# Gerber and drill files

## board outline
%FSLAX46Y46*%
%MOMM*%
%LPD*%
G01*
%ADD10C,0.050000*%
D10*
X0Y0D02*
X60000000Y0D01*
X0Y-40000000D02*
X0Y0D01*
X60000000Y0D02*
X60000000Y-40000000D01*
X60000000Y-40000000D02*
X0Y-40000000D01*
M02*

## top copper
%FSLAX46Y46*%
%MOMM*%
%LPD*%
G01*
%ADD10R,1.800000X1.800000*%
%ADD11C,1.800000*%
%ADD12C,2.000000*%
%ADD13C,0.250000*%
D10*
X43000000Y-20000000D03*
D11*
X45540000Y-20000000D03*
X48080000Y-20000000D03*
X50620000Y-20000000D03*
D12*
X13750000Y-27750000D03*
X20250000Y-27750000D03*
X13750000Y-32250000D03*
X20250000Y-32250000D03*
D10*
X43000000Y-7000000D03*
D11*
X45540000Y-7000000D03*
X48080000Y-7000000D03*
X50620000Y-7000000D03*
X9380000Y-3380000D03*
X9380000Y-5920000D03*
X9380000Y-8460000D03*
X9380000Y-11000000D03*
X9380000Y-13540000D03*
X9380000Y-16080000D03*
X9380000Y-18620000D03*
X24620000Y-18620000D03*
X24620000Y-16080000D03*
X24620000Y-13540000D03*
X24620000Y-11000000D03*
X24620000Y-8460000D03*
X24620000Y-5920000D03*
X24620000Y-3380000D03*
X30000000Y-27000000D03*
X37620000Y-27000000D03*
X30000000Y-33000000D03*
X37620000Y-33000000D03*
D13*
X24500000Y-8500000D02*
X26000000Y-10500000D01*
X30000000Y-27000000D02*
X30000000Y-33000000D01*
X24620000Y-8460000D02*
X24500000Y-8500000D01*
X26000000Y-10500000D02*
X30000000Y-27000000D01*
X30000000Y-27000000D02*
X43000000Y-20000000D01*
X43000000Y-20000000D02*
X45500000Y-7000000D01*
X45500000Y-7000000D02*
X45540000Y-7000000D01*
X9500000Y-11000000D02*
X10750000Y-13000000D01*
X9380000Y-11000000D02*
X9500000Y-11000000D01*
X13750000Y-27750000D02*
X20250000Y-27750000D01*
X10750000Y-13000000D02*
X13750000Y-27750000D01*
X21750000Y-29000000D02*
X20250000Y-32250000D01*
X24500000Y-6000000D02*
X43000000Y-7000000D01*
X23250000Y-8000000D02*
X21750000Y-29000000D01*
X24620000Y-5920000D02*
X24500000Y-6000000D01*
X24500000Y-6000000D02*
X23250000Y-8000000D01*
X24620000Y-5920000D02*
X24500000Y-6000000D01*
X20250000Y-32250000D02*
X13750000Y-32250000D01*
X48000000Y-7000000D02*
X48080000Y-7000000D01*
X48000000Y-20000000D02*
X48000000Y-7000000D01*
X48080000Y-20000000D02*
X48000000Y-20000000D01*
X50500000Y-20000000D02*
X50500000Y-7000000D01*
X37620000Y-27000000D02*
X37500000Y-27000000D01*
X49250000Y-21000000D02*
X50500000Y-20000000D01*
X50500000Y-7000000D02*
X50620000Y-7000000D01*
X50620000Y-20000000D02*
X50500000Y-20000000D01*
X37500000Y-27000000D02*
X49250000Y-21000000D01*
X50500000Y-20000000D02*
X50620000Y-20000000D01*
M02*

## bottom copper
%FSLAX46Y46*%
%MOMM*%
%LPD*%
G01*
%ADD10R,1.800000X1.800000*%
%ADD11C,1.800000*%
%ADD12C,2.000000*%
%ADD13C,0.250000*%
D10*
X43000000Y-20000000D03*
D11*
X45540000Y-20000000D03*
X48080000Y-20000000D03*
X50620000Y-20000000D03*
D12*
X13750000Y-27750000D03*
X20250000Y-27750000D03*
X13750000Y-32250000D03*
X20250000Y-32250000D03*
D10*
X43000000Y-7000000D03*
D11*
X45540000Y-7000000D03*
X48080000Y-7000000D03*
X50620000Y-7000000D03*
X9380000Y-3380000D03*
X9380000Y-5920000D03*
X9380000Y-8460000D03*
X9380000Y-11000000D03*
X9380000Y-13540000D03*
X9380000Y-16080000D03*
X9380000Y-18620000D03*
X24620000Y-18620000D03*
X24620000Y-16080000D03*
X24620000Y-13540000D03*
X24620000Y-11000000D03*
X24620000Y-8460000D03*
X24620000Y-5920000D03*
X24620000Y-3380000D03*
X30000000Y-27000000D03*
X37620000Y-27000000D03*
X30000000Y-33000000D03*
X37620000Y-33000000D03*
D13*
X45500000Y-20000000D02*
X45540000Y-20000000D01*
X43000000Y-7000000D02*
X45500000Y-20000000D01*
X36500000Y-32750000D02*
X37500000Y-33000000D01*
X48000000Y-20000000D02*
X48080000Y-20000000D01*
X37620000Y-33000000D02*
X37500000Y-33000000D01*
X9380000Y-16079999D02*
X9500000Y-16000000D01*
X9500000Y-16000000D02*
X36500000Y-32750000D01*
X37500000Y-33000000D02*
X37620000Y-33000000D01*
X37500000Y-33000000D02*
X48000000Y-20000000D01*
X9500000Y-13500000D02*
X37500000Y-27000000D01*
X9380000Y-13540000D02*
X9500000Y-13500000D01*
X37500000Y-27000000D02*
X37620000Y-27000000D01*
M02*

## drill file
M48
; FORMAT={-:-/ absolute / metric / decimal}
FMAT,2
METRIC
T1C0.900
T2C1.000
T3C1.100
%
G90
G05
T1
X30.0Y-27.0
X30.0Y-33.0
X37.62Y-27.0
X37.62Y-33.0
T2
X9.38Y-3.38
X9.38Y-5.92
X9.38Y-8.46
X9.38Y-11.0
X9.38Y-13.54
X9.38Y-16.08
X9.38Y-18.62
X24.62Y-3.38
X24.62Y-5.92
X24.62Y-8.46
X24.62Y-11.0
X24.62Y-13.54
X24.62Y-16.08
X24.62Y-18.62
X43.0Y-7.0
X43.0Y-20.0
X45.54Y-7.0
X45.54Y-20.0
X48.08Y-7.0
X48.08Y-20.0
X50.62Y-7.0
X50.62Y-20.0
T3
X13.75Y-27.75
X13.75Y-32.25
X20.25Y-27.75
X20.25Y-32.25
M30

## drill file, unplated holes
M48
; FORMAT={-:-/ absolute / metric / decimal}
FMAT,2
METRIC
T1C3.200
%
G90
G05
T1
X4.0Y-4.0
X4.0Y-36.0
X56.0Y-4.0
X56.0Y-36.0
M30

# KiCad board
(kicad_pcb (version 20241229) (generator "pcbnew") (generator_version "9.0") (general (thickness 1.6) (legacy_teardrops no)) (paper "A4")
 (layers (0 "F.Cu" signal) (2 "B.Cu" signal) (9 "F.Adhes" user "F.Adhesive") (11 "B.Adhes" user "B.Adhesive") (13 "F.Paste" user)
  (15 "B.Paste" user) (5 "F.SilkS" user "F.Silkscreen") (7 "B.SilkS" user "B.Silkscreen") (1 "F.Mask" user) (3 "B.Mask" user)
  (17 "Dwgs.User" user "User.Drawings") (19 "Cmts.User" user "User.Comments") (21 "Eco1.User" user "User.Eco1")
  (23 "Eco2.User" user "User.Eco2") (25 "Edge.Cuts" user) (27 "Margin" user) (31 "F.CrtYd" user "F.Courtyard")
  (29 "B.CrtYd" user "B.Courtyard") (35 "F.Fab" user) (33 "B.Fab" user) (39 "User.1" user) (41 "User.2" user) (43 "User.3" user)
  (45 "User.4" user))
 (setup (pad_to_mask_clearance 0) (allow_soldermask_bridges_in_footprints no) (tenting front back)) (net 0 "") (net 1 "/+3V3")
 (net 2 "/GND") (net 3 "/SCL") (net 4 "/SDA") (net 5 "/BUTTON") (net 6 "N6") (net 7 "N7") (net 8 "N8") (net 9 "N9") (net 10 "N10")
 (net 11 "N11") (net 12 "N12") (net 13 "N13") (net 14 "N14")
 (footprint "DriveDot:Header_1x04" (layer "F.Cu") (at 43 20)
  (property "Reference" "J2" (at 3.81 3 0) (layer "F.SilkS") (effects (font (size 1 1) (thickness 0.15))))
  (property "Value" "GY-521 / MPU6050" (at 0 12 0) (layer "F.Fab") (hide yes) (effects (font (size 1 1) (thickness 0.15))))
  (pad "1" thru_hole rect (at 0 0) (size 1.8 1.8) (drill 1) (layers "*.Cu" "*.Mask") (remove_unused_layers no) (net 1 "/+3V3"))
  (pad "2" thru_hole circle (at 2.54 0) (size 1.8 1.8) (drill 1) (layers "*.Cu" "*.Mask") (remove_unused_layers no) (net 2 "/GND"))
  (pad "3" thru_hole circle (at 5.08 0) (size 1.8 1.8) (drill 1) (layers "*.Cu" "*.Mask") (remove_unused_layers no) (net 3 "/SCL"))
  (pad "4" thru_hole circle (at 7.62 0) (size 1.8 1.8) (drill 1) (layers "*.Cu" "*.Mask") (remove_unused_layers no) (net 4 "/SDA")))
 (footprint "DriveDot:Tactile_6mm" (layer "F.Cu") (at 17 30)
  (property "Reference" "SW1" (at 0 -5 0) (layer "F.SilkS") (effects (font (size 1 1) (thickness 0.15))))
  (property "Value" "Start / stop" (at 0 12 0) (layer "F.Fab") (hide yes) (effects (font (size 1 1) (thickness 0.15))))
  (pad "1" thru_hole circle (at -3.25 -2.25) (size 2 2) (drill 1.1) (layers "*.Cu" "*.Mask") (remove_unused_layers no) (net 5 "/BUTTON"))
  (pad "1" thru_hole circle (at 3.25 -2.25) (size 2 2) (drill 1.1) (layers "*.Cu" "*.Mask") (remove_unused_layers no) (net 5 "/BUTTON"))
  (pad "2" thru_hole circle (at -3.25 2.25) (size 2 2) (drill 1.1) (layers "*.Cu" "*.Mask") (remove_unused_layers no) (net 2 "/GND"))
  (pad "2" thru_hole circle (at 3.25 2.25) (size 2 2) (drill 1.1) (layers "*.Cu" "*.Mask") (remove_unused_layers no) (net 2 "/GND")))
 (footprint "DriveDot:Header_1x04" (layer "F.Cu") (at 43 7)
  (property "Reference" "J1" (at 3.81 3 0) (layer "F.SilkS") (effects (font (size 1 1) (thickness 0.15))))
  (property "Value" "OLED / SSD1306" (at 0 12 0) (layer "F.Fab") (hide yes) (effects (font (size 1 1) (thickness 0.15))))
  (pad "1" thru_hole rect (at 0 0) (size 1.8 1.8) (drill 1) (layers "*.Cu" "*.Mask") (remove_unused_layers no) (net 2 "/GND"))
  (pad "2" thru_hole circle (at 2.54 0) (size 1.8 1.8) (drill 1) (layers "*.Cu" "*.Mask") (remove_unused_layers no) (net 1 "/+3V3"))
  (pad "3" thru_hole circle (at 5.08 0) (size 1.8 1.8) (drill 1) (layers "*.Cu" "*.Mask") (remove_unused_layers no) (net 3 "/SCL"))
  (pad "4" thru_hole circle (at 7.62 0) (size 1.8 1.8) (drill 1) (layers "*.Cu" "*.Mask") (remove_unused_layers no) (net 4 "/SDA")))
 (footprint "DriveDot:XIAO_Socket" (layer "F.Cu") (at 17 11)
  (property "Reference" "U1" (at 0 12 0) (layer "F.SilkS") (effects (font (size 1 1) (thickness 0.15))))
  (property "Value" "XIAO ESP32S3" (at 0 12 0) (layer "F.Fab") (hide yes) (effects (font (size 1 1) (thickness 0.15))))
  (pad "1" thru_hole circle (at -7.62 -7.62) (size 1.8 1.8) (drill 1) (layers "*.Cu" "*.Mask") (remove_unused_layers no) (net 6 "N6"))
  (pad "2" thru_hole circle (at -7.62 -5.08) (size 1.8 1.8) (drill 1) (layers "*.Cu" "*.Mask") (remove_unused_layers no) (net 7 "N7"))
  (pad "3" thru_hole circle (at -7.62 -2.54) (size 1.8 1.8) (drill 1) (layers "*.Cu" "*.Mask") (remove_unused_layers no) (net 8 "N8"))
  (pad "4" thru_hole circle (at -7.62 0) (size 1.8 1.8) (drill 1) (layers "*.Cu" "*.Mask") (remove_unused_layers no) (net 5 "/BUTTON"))
  (pad "5" thru_hole circle (at -7.62 2.54) (size 1.8 1.8) (drill 1) (layers "*.Cu" "*.Mask") (remove_unused_layers no) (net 4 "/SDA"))
  (pad "6" thru_hole circle (at -7.62 5.08) (size 1.8 1.8) (drill 1) (layers "*.Cu" "*.Mask") (remove_unused_layers no) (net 3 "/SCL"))
  (pad "7" thru_hole circle (at -7.62 7.62) (size 1.8 1.8) (drill 1) (layers "*.Cu" "*.Mask") (remove_unused_layers no) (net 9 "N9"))
  (pad "8" thru_hole circle (at 7.62 7.62) (size 1.8 1.8) (drill 1) (layers "*.Cu" "*.Mask") (remove_unused_layers no) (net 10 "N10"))
  (pad "9" thru_hole circle (at 7.62 5.08) (size 1.8 1.8) (drill 1) (layers "*.Cu" "*.Mask") (remove_unused_layers no) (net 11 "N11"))
  (pad "10" thru_hole circle (at 7.62 2.54) (size 1.8 1.8) (drill 1) (layers "*.Cu" "*.Mask") (remove_unused_layers no) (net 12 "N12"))
  (pad "11" thru_hole circle (at 7.62 0) (size 1.8 1.8) (drill 1) (layers "*.Cu" "*.Mask") (remove_unused_layers no) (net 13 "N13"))
  (pad "12" thru_hole circle (at 7.62 -2.54) (size 1.8 1.8) (drill 1) (layers "*.Cu" "*.Mask") (remove_unused_layers no) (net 1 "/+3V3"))
  (pad "13" thru_hole circle (at 7.62 -5.08) (size 1.8 1.8) (drill 1) (layers "*.Cu" "*.Mask") (remove_unused_layers no) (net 2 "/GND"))
  (pad "14" thru_hole circle (at 7.62 -7.62) (size 1.8 1.8) (drill 1) (layers "*.Cu" "*.Mask") (remove_unused_layers no) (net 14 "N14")))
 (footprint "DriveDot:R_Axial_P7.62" (layer "F.Cu") (at 30 27)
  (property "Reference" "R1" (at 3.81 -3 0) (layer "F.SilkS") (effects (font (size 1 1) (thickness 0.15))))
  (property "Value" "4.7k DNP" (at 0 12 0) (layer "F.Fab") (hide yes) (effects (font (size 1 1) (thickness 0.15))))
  (pad "1" thru_hole circle (at 0 0) (size 1.8 1.8) (drill 0.9) (layers "*.Cu" "*.Mask") (remove_unused_layers no) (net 1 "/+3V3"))
  (pad "2" thru_hole circle (at 7.62 0) (size 1.8 1.8) (drill 0.9) (layers "*.Cu" "*.Mask") (remove_unused_layers no) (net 4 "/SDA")))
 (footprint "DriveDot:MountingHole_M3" (layer "F.Cu") (at 4 4)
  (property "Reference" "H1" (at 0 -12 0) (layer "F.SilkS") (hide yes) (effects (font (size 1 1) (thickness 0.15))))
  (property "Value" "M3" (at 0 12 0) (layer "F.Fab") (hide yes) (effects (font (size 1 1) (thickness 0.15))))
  (pad "" np_thru_hole circle (at 0 0) (size 3.2 3.2) (drill 3.2) (layers "*.Cu" "*.Mask")))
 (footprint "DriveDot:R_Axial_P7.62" (layer "F.Cu") (at 30 33)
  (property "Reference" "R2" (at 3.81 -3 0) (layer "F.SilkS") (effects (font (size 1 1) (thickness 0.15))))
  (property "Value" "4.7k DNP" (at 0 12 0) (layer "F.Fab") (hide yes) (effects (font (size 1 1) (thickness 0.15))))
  (pad "1" thru_hole circle (at 0 0) (size 1.8 1.8) (drill 0.9) (layers "*.Cu" "*.Mask") (remove_unused_layers no) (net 1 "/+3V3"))
  (pad "2" thru_hole circle (at 7.62 0) (size 1.8 1.8) (drill 0.9) (layers "*.Cu" "*.Mask") (remove_unused_layers no) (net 3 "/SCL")))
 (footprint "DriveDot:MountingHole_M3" (layer "F.Cu") (at 4 36)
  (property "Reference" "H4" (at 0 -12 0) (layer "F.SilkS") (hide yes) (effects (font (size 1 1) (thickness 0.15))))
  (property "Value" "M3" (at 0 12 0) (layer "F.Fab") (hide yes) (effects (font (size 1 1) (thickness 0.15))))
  (pad "" np_thru_hole circle (at 0 0) (size 3.2 3.2) (drill 3.2) (layers "*.Cu" "*.Mask")))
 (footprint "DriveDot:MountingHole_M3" (layer "F.Cu") (at 56 4)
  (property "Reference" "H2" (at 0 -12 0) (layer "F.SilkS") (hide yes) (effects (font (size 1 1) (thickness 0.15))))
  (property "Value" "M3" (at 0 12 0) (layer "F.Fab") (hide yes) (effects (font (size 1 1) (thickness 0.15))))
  (pad "" np_thru_hole circle (at 0 0) (size 3.2 3.2) (drill 3.2) (layers "*.Cu" "*.Mask")))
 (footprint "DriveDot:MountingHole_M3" (layer "F.Cu") (at 56 36)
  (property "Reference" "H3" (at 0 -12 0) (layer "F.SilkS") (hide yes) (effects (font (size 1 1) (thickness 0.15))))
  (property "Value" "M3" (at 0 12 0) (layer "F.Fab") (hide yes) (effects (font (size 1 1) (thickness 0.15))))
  (pad "" np_thru_hole circle (at 0 0) (size 3.2 3.2) (drill 3.2) (layers "*.Cu" "*.Mask")))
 (gr_line (start 0 0) (end 60 0) (stroke (width 0.05) (type default)) (layer "Edge.Cuts"))
 (gr_line (start 0 40) (end 0 0) (stroke (width 0.05) (type default)) (layer "Edge.Cuts"))
 (gr_line (start 60 0) (end 60 40) (stroke (width 0.05) (type default)) (layer "Edge.Cuts"))
 (gr_line (start 60 40) (end 0 40) (stroke (width 0.05) (type default)) (layer "Edge.Cuts"))
 (segment (start 24.5 8.5) (end 26 10.5) (width 0.25) (layer "F.Cu") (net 1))
 (segment (start 30 27) (end 30 33) (width 0.25) (layer "F.Cu") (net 1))
 (segment (start 24.62 8.46) (end 24.5 8.5) (width 0.25) (layer "F.Cu") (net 1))
 (segment (start 26 10.5) (end 30 27) (width 0.25) (layer "F.Cu") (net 1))
 (segment (start 30 27) (end 43 20) (width 0.25) (layer "F.Cu") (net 1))
 (segment (start 43 20) (end 45.5 7) (width 0.25) (layer "F.Cu") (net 1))
 (segment (start 45.5 7) (end 45.54 7) (width 0.25) (layer "F.Cu") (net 1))
 (segment (start 9.5 11) (end 10.75 13) (width 0.25) (layer "F.Cu") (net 5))
 (segment (start 9.38 11) (end 9.5 11) (width 0.25) (layer "F.Cu") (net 5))
 (segment (start 13.75 27.75) (end 20.25 27.75) (width 0.25) (layer "F.Cu") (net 5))
 (segment (start 10.75 13) (end 13.75 27.75) (width 0.25) (layer "F.Cu") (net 5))
 (segment (start 21.75 29) (end 20.25 32.25) (width 0.25) (layer "F.Cu") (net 2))
 (segment (start 24.5 6) (end 43 7) (width 0.25) (layer "F.Cu") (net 2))
 (segment (start 23.25 8) (end 21.75 29) (width 0.25) (layer "F.Cu") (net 2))
 (segment (start 24.62 5.92) (end 24.5 6) (width 0.25) (layer "F.Cu") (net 2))
 (segment (start 24.5 6) (end 23.25 8) (width 0.25) (layer "F.Cu") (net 2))
 (segment (start 24.62 5.92) (end 24.5 6) (width 0.25) (layer "F.Cu") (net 2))
 (segment (start 20.25 32.25) (end 13.75 32.25) (width 0.25) (layer "F.Cu") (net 2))
 (segment (start 45.5 20) (end 45.54 20) (width 0.25) (layer "B.Cu") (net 2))
 (segment (start 43 7) (end 45.5 20) (width 0.25) (layer "B.Cu") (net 2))
 (segment (start 48 7) (end 48.08 7) (width 0.25) (layer "F.Cu") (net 3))
 (segment (start 48 20) (end 48 7) (width 0.25) (layer "F.Cu") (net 3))
 (segment (start 48.08 20) (end 48 20) (width 0.25) (layer "F.Cu") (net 3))
 (segment (start 36.5 32.75) (end 37.5 33) (width 0.25) (layer "B.Cu") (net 3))
 (segment (start 48 20) (end 48.08 20) (width 0.25) (layer "B.Cu") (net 3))
 (segment (start 37.62 33) (end 37.5 33) (width 0.25) (layer "B.Cu") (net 3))
 (segment (start 9.38 16.079999) (end 9.5 16) (width 0.25) (layer "B.Cu") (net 3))
 (segment (start 9.5 16) (end 36.5 32.75) (width 0.25) (layer "B.Cu") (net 3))
 (segment (start 37.5 33) (end 37.62 33) (width 0.25) (layer "B.Cu") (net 3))
 (segment (start 37.5 33) (end 48 20) (width 0.25) (layer "B.Cu") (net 3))
 (segment (start 50.5 20) (end 50.5 7) (width 0.25) (layer "F.Cu") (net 4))
 (segment (start 37.62 27) (end 37.5 27) (width 0.25) (layer "F.Cu") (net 4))
 (segment (start 49.25 21) (end 50.5 20) (width 0.25) (layer "F.Cu") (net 4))
 (segment (start 50.5 7) (end 50.62 7) (width 0.25) (layer "F.Cu") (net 4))
 (segment (start 50.62 20) (end 50.5 20) (width 0.25) (layer "F.Cu") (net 4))
 (segment (start 37.5 27) (end 49.25 21) (width 0.25) (layer "F.Cu") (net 4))
 (segment (start 50.5 20) (end 50.62 20) (width 0.25) (layer "F.Cu") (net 4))
 (segment (start 9.5 13.5) (end 37.5 27) (width 0.25) (layer "B.Cu") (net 4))
 (segment (start 9.38 13.54) (end 9.5 13.5) (width 0.25) (layer "B.Cu") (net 4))
 (segment (start 37.5 27) (end 37.62 27) (width 0.25) (layer "B.Cu") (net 4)))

